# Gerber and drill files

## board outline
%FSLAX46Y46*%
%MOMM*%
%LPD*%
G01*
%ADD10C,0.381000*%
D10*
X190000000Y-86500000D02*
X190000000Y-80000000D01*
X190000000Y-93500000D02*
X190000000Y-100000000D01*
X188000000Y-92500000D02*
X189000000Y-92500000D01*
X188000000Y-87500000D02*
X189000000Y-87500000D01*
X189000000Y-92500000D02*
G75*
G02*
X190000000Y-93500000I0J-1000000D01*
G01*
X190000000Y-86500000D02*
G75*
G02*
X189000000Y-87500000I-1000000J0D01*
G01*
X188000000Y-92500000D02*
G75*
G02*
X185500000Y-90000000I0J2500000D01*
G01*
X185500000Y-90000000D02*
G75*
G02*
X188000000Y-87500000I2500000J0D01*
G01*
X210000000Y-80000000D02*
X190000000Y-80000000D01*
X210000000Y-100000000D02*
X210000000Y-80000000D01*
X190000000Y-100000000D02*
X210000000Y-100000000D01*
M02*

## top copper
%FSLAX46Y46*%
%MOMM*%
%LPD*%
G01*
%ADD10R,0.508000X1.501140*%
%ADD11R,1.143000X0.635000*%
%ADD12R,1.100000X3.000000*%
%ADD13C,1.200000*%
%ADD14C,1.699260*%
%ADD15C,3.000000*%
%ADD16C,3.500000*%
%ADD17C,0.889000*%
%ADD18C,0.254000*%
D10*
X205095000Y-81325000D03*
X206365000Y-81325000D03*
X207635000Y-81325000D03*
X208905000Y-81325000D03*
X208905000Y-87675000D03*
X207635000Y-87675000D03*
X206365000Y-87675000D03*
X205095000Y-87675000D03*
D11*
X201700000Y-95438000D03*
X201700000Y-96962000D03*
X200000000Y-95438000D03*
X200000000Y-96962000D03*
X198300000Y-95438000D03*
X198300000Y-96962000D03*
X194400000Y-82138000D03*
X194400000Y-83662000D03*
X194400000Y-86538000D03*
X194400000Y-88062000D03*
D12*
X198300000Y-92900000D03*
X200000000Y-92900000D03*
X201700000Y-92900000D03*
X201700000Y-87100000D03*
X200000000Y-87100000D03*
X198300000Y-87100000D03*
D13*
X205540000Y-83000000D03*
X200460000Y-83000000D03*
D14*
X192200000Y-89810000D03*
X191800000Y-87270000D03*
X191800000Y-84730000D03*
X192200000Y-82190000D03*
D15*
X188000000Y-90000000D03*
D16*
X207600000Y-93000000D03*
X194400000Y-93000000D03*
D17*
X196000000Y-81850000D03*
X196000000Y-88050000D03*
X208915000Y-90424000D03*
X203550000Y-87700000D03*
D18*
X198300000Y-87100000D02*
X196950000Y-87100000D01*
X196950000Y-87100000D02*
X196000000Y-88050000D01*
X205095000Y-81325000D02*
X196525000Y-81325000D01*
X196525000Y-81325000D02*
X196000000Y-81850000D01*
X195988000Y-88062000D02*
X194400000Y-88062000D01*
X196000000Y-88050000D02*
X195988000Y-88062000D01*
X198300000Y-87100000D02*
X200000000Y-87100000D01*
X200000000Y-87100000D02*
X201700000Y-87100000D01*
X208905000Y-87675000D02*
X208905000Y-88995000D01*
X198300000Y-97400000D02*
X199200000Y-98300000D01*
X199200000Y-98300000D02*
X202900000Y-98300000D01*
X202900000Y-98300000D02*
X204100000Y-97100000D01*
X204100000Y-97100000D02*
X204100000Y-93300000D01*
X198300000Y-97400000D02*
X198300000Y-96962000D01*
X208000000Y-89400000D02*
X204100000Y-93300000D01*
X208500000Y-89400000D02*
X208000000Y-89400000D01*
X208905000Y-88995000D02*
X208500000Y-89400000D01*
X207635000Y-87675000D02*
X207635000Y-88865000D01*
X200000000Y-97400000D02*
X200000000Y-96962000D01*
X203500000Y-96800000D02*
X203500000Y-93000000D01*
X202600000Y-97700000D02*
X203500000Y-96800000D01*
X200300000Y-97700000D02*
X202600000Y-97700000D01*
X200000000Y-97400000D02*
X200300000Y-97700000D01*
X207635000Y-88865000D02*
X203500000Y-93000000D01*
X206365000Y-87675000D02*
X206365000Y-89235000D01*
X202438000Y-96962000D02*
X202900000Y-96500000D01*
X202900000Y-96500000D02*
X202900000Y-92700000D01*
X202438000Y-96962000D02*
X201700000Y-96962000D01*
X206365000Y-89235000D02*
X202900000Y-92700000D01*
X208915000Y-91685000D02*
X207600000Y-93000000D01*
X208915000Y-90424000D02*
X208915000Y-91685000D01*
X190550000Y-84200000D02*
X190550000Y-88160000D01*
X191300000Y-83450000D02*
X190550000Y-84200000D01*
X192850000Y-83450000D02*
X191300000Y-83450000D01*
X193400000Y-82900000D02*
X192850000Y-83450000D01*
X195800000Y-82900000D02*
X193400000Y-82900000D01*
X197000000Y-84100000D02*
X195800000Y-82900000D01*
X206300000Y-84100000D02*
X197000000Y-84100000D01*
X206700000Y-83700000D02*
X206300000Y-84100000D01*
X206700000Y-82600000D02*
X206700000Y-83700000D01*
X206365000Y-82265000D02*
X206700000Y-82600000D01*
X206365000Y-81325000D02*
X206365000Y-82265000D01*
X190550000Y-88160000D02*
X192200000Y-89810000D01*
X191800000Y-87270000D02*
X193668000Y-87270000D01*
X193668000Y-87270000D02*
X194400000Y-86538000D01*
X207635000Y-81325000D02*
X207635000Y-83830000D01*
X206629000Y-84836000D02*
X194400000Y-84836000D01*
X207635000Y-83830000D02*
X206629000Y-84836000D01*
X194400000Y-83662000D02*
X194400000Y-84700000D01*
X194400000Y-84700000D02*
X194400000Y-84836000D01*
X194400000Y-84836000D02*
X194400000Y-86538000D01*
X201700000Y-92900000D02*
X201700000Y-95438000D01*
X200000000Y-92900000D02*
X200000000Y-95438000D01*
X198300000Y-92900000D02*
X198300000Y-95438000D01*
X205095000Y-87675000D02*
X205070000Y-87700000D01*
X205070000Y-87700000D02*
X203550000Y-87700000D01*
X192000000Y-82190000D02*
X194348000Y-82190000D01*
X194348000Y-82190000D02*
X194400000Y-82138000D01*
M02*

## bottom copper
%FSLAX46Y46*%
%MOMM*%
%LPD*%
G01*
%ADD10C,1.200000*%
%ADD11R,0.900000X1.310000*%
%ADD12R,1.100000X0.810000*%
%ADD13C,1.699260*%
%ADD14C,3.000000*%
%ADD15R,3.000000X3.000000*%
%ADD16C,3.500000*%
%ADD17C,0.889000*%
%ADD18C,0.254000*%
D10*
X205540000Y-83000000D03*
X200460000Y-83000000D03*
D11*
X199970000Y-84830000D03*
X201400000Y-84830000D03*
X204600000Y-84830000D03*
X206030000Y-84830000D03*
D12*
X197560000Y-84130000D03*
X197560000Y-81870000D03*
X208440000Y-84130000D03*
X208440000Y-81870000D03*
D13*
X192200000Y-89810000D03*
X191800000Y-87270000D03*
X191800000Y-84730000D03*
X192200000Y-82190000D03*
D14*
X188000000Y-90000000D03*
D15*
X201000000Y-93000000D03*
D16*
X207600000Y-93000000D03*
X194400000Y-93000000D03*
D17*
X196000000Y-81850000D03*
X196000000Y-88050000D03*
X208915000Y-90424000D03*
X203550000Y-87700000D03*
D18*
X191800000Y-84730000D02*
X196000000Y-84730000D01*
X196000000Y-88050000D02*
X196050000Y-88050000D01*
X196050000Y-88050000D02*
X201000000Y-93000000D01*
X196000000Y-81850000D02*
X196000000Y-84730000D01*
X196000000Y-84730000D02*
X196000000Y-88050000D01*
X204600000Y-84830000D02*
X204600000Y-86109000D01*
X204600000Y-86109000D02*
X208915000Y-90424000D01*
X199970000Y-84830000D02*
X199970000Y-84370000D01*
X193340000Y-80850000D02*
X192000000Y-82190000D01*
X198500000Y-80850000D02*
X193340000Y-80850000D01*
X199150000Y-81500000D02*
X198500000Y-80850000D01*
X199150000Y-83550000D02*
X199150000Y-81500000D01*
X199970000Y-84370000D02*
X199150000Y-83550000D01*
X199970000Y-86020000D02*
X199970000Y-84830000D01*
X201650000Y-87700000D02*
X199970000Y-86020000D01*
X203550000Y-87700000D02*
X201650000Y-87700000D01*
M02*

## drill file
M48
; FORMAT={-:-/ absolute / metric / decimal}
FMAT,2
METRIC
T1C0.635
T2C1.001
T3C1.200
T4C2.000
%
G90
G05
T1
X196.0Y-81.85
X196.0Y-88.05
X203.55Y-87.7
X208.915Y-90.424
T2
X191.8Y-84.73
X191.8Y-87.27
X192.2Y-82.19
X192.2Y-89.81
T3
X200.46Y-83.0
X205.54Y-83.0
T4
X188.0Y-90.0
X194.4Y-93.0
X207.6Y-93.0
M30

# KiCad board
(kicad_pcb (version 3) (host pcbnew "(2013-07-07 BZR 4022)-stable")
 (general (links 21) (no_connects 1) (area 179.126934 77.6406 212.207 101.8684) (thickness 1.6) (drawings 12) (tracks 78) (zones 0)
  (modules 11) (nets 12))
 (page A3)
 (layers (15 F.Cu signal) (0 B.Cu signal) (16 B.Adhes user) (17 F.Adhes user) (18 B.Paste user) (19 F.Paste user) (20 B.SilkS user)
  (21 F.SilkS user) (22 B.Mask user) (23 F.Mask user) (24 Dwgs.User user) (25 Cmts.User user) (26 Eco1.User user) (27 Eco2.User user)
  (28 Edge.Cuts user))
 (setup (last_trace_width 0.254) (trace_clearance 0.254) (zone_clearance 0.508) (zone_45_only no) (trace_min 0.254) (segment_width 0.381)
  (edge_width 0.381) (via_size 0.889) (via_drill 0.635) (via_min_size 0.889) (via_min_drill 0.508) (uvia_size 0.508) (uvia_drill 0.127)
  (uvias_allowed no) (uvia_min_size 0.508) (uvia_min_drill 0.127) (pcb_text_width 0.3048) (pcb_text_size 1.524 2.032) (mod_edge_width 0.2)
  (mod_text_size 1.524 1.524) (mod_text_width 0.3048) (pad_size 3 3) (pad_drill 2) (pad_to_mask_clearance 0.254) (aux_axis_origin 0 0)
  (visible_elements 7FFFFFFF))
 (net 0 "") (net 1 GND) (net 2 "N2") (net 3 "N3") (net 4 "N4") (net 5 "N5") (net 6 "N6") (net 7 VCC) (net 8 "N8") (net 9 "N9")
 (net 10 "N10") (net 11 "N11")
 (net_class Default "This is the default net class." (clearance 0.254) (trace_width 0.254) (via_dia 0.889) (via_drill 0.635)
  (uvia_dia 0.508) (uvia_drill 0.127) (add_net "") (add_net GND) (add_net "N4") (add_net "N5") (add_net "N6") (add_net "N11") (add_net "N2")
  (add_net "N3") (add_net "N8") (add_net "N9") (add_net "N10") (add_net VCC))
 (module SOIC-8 (layer F.Cu) (at 207 84.5)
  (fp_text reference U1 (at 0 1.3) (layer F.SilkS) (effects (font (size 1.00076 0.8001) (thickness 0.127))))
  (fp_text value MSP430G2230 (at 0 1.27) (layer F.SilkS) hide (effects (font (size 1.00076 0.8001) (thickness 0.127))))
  (pad 8 smd rect (at -1.905 -3.175) (size 0.508 1.50114) (layers F.Cu F.Paste F.Mask) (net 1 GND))
  (pad 7 smd rect (at -0.635 -3.175) (size 0.508 1.50114) (layers F.Cu F.Paste F.Mask) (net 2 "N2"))
  (pad 6 smd rect (at 0.635 -3.175) (size 0.508 1.50114) (layers F.Cu F.Paste F.Mask) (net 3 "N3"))
  (pad 5 smd rect (at 1.905 -3.175) (size 0.508 1.50114) (layers F.Cu F.Paste F.Mask))
  (pad 4 smd rect (at 1.905 3.175) (size 0.508 1.50114) (layers F.Cu F.Paste F.Mask) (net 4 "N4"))
  (pad 3 smd rect (at 0.635 3.175) (size 0.508 1.50114) (layers F.Cu F.Paste F.Mask) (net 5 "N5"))
  (pad 2 smd rect (at -0.635 3.175) (size 0.508 1.50114) (layers F.Cu F.Paste F.Mask) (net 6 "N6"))
  (pad 1 smd rect (at -1.905 3.175) (size 0.508 1.50114) (layers F.Cu F.Paste F.Mask) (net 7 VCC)))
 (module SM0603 (layer F.Cu) (at 201.7 96.2 270)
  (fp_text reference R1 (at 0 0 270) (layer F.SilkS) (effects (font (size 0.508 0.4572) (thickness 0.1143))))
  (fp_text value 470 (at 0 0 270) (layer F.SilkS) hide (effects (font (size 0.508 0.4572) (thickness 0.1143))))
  (pad 1 smd rect (at -0.762 0 270) (size 0.635 1.143) (layers F.Cu F.Paste F.Mask) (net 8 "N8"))
  (pad 2 smd rect (at 0.762 0 270) (size 0.635 1.143) (layers F.Cu F.Paste F.Mask) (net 6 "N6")))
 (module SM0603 (layer F.Cu) (at 200 96.2 270)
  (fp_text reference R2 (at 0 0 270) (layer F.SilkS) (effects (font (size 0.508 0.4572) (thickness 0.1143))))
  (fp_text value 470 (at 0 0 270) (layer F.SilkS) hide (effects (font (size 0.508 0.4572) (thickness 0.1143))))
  (pad 1 smd rect (at -0.762 0 270) (size 0.635 1.143) (layers F.Cu F.Paste F.Mask) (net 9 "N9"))
  (pad 2 smd rect (at 0.762 0 270) (size 0.635 1.143) (layers F.Cu F.Paste F.Mask) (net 5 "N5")))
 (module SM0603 (layer F.Cu) (at 198.3 96.2 270)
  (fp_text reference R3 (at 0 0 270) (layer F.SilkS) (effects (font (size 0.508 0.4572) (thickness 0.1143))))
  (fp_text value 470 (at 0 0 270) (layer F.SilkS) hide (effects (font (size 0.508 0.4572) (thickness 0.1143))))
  (pad 1 smd rect (at -0.762 0 270) (size 0.635 1.143) (layers F.Cu F.Paste F.Mask) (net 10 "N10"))
  (pad 2 smd rect (at 0.762 0 270) (size 0.635 1.143) (layers F.Cu F.Paste F.Mask) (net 4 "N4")))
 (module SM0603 (layer F.Cu) (at 194.4 82.9 270)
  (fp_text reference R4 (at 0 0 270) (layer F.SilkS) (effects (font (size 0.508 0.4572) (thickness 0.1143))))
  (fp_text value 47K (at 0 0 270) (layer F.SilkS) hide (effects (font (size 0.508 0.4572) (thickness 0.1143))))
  (pad 1 smd rect (at -0.762 0 270) (size 0.635 1.143) (layers F.Cu F.Paste F.Mask) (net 7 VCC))
  (pad 2 smd rect (at 0.762 0 270) (size 0.635 1.143) (layers F.Cu F.Paste F.Mask) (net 3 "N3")))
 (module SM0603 (layer F.Cu) (at 194.4 87.3 270)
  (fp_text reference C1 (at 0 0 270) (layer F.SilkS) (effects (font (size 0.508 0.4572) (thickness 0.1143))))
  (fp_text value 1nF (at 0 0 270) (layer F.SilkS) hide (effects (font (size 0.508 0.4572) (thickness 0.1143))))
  (pad 1 smd rect (at -0.762 0 270) (size 0.635 1.143) (layers F.Cu F.Paste F.Mask) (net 3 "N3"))
  (pad 2 smd rect (at 0.762 0 270) (size 0.635 1.143) (layers F.Cu F.Paste F.Mask) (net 1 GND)))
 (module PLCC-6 (layer F.Cu) (at 200 90)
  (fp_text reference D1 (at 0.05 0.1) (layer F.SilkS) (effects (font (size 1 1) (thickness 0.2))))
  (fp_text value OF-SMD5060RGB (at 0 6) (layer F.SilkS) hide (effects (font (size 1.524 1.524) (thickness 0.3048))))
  (pad 1 smd rect (at -1.7 2.9) (size 1.1 3) (layers F.Cu F.Paste F.Mask) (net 10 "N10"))
  (pad 2 smd rect (at 0 2.9) (size 1.1 3) (layers F.Cu F.Paste F.Mask) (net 9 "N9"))
  (pad 3 smd rect (at 1.7 2.9) (size 1.1 3) (layers F.Cu F.Paste F.Mask) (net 8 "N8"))
  (pad 4 smd rect (at 1.7 -2.9) (size 1.1 3) (layers F.Cu F.Paste F.Mask) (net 1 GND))
  (pad 5 smd rect (at 0 -2.9) (size 1.1 3) (layers F.Cu F.Paste F.Mask) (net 1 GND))
  (pad 6 smd rect (at -1.7 -2.9) (size 1.1 3) (layers F.Cu F.Paste F.Mask) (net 1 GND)))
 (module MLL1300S (layer B.Cu) (at 203 83)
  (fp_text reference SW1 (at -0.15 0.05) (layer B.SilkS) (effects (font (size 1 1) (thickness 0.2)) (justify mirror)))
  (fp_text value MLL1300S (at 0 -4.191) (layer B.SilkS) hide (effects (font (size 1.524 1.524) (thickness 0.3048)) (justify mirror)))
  (pad ~ thru_hole circle (at 2.54 0) (size 1.2 1.2) (drill 1.2) (layers *.Cu *.Mask B.SilkS))
  (pad ~ thru_hole circle (at -2.54 0) (size 1.2 1.2) (drill 1.2) (layers *.Cu *.Mask B.SilkS))
  (pad 1 smd rect (at -3.03 1.83) (size 0.9 1.31) (layers B.Cu B.Paste B.Mask) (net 7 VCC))
  (pad 2 smd rect (at -1.6 1.83) (size 0.9 1.31) (layers B.Cu B.Paste B.Mask))
  (pad 3 smd rect (at 1.6 1.83) (size 0.9 1.31) (layers B.Cu B.Paste B.Mask) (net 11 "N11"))
  (pad 4 smd rect (at 3.03 1.83) (size 0.9 1.31) (layers B.Cu B.Paste B.Mask))
  (pad ~ smd rect (at -5.44 1.13) (size 1.1 0.81) (layers B.Cu B.Paste B.Mask))
  (pad ~ smd rect (at -5.44 -1.13) (size 1.1 0.81) (layers B.Cu B.Paste B.Mask))
  (pad ~ smd rect (at 5.44 1.13) (size 1.1 0.81) (layers B.Cu B.Paste B.Mask))
  (pad ~ smd rect (at 5.44 -1.13) (size 1.1 0.81) (layers B.Cu B.Paste B.Mask)))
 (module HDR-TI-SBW (layer F.Cu) (at 192 86 90)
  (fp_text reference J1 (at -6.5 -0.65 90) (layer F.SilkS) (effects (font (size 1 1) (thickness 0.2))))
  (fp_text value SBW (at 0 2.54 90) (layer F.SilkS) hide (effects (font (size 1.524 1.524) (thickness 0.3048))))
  (pad 1 thru_hole circle (at -3.81 0.2 90) (size 1.69926 1.69926) (drill 1.00076) (layers *.Cu *.Mask F.SilkS) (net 2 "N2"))
  (pad 2 thru_hole circle (at -1.27 -0.2 90) (size 1.69926 1.69926) (drill 1.00076) (layers *.Cu *.Mask F.SilkS) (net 3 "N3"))
  (pad 3 thru_hole circle (at 1.27 -0.2 90) (size 1.69926 1.69926) (drill 1.00076) (layers *.Cu *.Mask F.SilkS) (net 1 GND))
  (pad 4 thru_hole circle (at 3.81 0.2 90) (size 1.69926 1.69926) (drill 1.00076) (layers *.Cu *.Mask F.SilkS) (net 7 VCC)))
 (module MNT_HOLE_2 (layer F.Cu) (at 188 90)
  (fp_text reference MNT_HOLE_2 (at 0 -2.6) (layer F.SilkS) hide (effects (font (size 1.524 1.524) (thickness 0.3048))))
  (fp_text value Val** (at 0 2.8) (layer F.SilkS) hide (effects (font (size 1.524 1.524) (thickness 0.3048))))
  (pad "" thru_hole circle (at 0 0) (size 3 3) (drill 2) (layers *.Cu *.Mask F.SilkS)))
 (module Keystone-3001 (layer B.Cu) (at 201 93)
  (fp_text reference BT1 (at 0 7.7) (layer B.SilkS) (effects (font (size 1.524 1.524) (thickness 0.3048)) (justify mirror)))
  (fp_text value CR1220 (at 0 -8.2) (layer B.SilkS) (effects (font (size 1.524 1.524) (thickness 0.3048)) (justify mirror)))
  (pad 2 smd rect (at 0 0) (size 3 3) (layers B.Cu B.Paste B.Mask) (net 1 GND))
  (pad 1 thru_hole circle (at 6.6 0) (size 3.5 3.5) (drill 2) (layers F.Cu F.Mask) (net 11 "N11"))
  (pad 1 thru_hole circle (at -6.6 0) (size 3.5 3.5) (drill 2) (layers F.Cu F.Mask) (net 11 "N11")))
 (gr_line (start 190 86.5) (end 190 80) (angle 90) (layer Edge.Cuts) (width 0.381))
 (gr_line (start 190 93.5) (end 190 100) (angle 90) (layer Edge.Cuts) (width 0.381))
 (gr_line (start 188 92.5) (end 189 92.5) (angle 90) (layer Edge.Cuts) (width 0.381))
 (gr_line (start 188 87.5) (end 189 87.5) (angle 90) (layer Edge.Cuts) (width 0.381))
 (gr_arc (start 189 93.5) (end 189 92.5) (angle 90) (layer Edge.Cuts) (width 0.381))
 (gr_arc (start 189 86.5) (end 190 86.5) (angle 90) (layer Edge.Cuts) (width 0.381))
 (gr_arc (start 188 90) (end 188 92.5) (angle 90) (layer Edge.Cuts) (width 0.381))
 (gr_arc (start 188 90) (end 185.5 90) (angle 90) (layer Edge.Cuts) (width 0.381))
 (gr_line (start 210 80) (end 190 80) (angle 90) (layer Edge.Cuts) (width 0.381))
 (gr_line (start 210 100) (end 210 80) (angle 90) (layer Edge.Cuts) (width 0.381))
 (gr_line (start 190 100) (end 210 100) (angle 90) (layer Edge.Cuts) (width 0.381))
 (segment (start 191.8 84.73) (end 196 84.73) (width 0.254) (layer B.Cu) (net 1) (status 400000))
 (segment (start 196 88.05) (end 196.05 88.05) (width 0.254) (layer B.Cu) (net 1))
 (segment (start 196.05 88.05) (end 201 93) (width 0.254) (layer B.Cu) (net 1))
 (segment (start 198.3 87.1) (end 196.95 87.1) (width 0.254) (layer F.Cu) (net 1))
 (segment (start 196.95 87.1) (end 196 88.05) (width 0.254) (layer F.Cu) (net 1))
 (segment (start 205.095 81.325) (end 196.525 81.325) (width 0.254) (layer F.Cu) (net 1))
 (segment (start 196.525 81.325) (end 196 81.85) (width 0.254) (layer F.Cu) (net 1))
 (via (at 196 81.85) (size 0.889) (layers F.Cu B.Cu) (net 1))
 (segment (start 196 81.85) (end 196 84.73) (width 0.254) (layer B.Cu) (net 1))
 (segment (start 196 84.73) (end 196 88.05) (width 0.254) (layer B.Cu) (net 1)) (via (at 196 88.05) (size 0.889) (layers F.Cu B.Cu) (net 1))
 (segment (start 195.988 88.062) (end 194.4 88.062) (width 0.254) (layer F.Cu) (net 1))
 (segment (start 196 88.05) (end 195.988 88.062) (width 0.254) (layer F.Cu) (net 1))
 (segment (start 198.3 87.1) (end 200 87.1) (width 0.254) (layer F.Cu) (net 1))
 (segment (start 200 87.1) (end 201.7 87.1) (width 0.254) (layer F.Cu) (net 1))
 (segment (start 208.905 87.675) (end 208.905 88.995) (width 0.254) (layer F.Cu) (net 4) (status 10))
 (segment (start 198.3 97.4) (end 199.2 98.3) (width 0.254) (layer F.Cu) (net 4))
 (segment (start 199.2 98.3) (end 202.9 98.3) (width 0.254) (layer F.Cu) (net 4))
 (segment (start 202.9 98.3) (end 204.1 97.1) (width 0.254) (layer F.Cu) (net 4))
 (segment (start 204.1 97.1) (end 204.1 93.3) (width 0.254) (layer F.Cu) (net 4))
 (segment (start 198.3 97.4) (end 198.3 96.962) (width 0.254) (layer F.Cu) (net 4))
 (segment (start 208 89.4) (end 204.1 93.3) (width 0.254) (layer F.Cu) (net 4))
 (segment (start 208.5 89.4) (end 208 89.4) (width 0.254) (layer F.Cu) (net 4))
 (segment (start 208.905 88.995) (end 208.5 89.4) (width 0.254) (layer F.Cu) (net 4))
 (segment (start 207.635 87.675) (end 207.635 88.865) (width 0.254) (layer F.Cu) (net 5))
 (segment (start 200 97.4) (end 200 96.962) (width 0.254) (layer F.Cu) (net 5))
 (segment (start 203.5 96.8) (end 203.5 93) (width 0.254) (layer F.Cu) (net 5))
 (segment (start 202.6 97.7) (end 203.5 96.8) (width 0.254) (layer F.Cu) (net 5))
 (segment (start 200.3 97.7) (end 202.6 97.7) (width 0.254) (layer F.Cu) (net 5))
 (segment (start 200 97.4) (end 200.3 97.7) (width 0.254) (layer F.Cu) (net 5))
 (segment (start 207.635 88.865) (end 203.5 93) (width 0.254) (layer F.Cu) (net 5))
 (segment (start 206.365 87.675) (end 206.365 89.235) (width 0.254) (layer F.Cu) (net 6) (status 10))
 (segment (start 202.438 96.962) (end 202.9 96.5) (width 0.254) (layer F.Cu) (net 6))
 (segment (start 202.9 96.5) (end 202.9 92.7) (width 0.254) (layer F.Cu) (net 6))
 (segment (start 202.438 96.962) (end 201.7 96.962) (width 0.254) (layer F.Cu) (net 6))
 (segment (start 206.365 89.235) (end 202.9 92.7) (width 0.254) (layer F.Cu) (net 6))
 (segment (start 204.6 84.83) (end 204.6 86.109) (width 0.254) (layer B.Cu) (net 11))
 (segment (start 208.915 91.685) (end 207.6 93) (width 0.254) (layer F.Cu) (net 11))
 (segment (start 208.915 90.424) (end 208.915 91.685) (width 0.254) (layer F.Cu) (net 11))
 (via (at 208.915 90.424) (size 0.889) (layers F.Cu B.Cu) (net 11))
 (segment (start 204.6 86.109) (end 208.915 90.424) (width 0.254) (layer B.Cu) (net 11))
 (segment (start 190.55 84.2) (end 190.55 88.16) (width 0.254) (layer F.Cu) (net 2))
 (segment (start 191.3 83.45) (end 190.55 84.2) (width 0.254) (layer F.Cu) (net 2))
 (segment (start 192.85 83.45) (end 191.3 83.45) (width 0.254) (layer F.Cu) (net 2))
 (segment (start 193.4 82.9) (end 192.85 83.45) (width 0.254) (layer F.Cu) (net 2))
 (segment (start 195.8 82.9) (end 193.4 82.9) (width 0.254) (layer F.Cu) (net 2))
 (segment (start 197 84.1) (end 195.8 82.9) (width 0.254) (layer F.Cu) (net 2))
 (segment (start 206.3 84.1) (end 197 84.1) (width 0.254) (layer F.Cu) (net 2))
 (segment (start 206.7 83.7) (end 206.3 84.1) (width 0.254) (layer F.Cu) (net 2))
 (segment (start 206.7 82.6) (end 206.7 83.7) (width 0.254) (layer F.Cu) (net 2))
 (segment (start 206.365 82.265) (end 206.7 82.6) (width 0.254) (layer F.Cu) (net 2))
 (segment (start 206.365 81.325) (end 206.365 82.265) (width 0.254) (layer F.Cu) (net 2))
 (segment (start 190.55 88.16) (end 192.2 89.81) (width 0.254) (layer F.Cu) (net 2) (status 800000))
 (segment (start 191.8 87.27) (end 193.668 87.27) (width 0.254) (layer F.Cu) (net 3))
 (segment (start 193.668 87.27) (end 194.4 86.538) (width 0.254) (layer F.Cu) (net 3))
 (segment (start 207.635 81.325) (end 207.635 83.83) (width 0.254) (layer F.Cu) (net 3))
 (segment (start 206.629 84.836) (end 194.4 84.836) (width 0.254) (layer F.Cu) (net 3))
 (segment (start 207.635 83.83) (end 206.629 84.836) (width 0.254) (layer F.Cu) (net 3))
 (segment (start 194.4 83.662) (end 194.4 84.7) (width 0.254) (layer F.Cu) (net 3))
 (segment (start 194.4 84.7) (end 194.4 84.836) (width 0.254) (layer F.Cu) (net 3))
 (segment (start 194.4 84.836) (end 194.4 86.538) (width 0.254) (layer F.Cu) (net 3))
 (segment (start 201.7 92.9) (end 201.7 95.438) (width 0.254) (layer F.Cu) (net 8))
 (segment (start 200 92.9) (end 200 95.438) (width 0.254) (layer F.Cu) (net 9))
 (segment (start 198.3 92.9) (end 198.3 95.438) (width 0.254) (layer F.Cu) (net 10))
 (segment (start 199.97 84.83) (end 199.97 84.37) (width 0.254) (layer B.Cu) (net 7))
 (segment (start 193.34 80.85) (end 192 82.19) (width 0.254) (layer B.Cu) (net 7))
 (segment (start 198.5 80.85) (end 193.34 80.85) (width 0.254) (layer B.Cu) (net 7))
 (segment (start 199.15 81.5) (end 198.5 80.85) (width 0.254) (layer B.Cu) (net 7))
 (segment (start 199.15 83.55) (end 199.15 81.5) (width 0.254) (layer B.Cu) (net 7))
 (segment (start 199.97 84.37) (end 199.15 83.55) (width 0.254) (layer B.Cu) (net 7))
 (segment (start 205.095 87.675) (end 205.07 87.7) (width 0.254) (layer F.Cu) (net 7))
 (segment (start 199.97 86.02) (end 199.97 84.83) (width 0.254) (layer B.Cu) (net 7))
 (segment (start 201.65 87.7) (end 199.97 86.02) (width 0.254) (layer B.Cu) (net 7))
 (segment (start 203.55 87.7) (end 201.65 87.7) (width 0.254) (layer B.Cu) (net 7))
 (via (at 203.55 87.7) (size 0.889) (layers F.Cu B.Cu) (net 7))
 (segment (start 205.07 87.7) (end 203.55 87.7) (width 0.254) (layer F.Cu) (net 7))
 (segment (start 192 82.19) (end 194.348 82.19) (width 0.254) (layer F.Cu) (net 7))
 (segment (start 194.348 82.19) (end 194.4 82.138) (width 0.254) (layer F.Cu) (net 7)))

